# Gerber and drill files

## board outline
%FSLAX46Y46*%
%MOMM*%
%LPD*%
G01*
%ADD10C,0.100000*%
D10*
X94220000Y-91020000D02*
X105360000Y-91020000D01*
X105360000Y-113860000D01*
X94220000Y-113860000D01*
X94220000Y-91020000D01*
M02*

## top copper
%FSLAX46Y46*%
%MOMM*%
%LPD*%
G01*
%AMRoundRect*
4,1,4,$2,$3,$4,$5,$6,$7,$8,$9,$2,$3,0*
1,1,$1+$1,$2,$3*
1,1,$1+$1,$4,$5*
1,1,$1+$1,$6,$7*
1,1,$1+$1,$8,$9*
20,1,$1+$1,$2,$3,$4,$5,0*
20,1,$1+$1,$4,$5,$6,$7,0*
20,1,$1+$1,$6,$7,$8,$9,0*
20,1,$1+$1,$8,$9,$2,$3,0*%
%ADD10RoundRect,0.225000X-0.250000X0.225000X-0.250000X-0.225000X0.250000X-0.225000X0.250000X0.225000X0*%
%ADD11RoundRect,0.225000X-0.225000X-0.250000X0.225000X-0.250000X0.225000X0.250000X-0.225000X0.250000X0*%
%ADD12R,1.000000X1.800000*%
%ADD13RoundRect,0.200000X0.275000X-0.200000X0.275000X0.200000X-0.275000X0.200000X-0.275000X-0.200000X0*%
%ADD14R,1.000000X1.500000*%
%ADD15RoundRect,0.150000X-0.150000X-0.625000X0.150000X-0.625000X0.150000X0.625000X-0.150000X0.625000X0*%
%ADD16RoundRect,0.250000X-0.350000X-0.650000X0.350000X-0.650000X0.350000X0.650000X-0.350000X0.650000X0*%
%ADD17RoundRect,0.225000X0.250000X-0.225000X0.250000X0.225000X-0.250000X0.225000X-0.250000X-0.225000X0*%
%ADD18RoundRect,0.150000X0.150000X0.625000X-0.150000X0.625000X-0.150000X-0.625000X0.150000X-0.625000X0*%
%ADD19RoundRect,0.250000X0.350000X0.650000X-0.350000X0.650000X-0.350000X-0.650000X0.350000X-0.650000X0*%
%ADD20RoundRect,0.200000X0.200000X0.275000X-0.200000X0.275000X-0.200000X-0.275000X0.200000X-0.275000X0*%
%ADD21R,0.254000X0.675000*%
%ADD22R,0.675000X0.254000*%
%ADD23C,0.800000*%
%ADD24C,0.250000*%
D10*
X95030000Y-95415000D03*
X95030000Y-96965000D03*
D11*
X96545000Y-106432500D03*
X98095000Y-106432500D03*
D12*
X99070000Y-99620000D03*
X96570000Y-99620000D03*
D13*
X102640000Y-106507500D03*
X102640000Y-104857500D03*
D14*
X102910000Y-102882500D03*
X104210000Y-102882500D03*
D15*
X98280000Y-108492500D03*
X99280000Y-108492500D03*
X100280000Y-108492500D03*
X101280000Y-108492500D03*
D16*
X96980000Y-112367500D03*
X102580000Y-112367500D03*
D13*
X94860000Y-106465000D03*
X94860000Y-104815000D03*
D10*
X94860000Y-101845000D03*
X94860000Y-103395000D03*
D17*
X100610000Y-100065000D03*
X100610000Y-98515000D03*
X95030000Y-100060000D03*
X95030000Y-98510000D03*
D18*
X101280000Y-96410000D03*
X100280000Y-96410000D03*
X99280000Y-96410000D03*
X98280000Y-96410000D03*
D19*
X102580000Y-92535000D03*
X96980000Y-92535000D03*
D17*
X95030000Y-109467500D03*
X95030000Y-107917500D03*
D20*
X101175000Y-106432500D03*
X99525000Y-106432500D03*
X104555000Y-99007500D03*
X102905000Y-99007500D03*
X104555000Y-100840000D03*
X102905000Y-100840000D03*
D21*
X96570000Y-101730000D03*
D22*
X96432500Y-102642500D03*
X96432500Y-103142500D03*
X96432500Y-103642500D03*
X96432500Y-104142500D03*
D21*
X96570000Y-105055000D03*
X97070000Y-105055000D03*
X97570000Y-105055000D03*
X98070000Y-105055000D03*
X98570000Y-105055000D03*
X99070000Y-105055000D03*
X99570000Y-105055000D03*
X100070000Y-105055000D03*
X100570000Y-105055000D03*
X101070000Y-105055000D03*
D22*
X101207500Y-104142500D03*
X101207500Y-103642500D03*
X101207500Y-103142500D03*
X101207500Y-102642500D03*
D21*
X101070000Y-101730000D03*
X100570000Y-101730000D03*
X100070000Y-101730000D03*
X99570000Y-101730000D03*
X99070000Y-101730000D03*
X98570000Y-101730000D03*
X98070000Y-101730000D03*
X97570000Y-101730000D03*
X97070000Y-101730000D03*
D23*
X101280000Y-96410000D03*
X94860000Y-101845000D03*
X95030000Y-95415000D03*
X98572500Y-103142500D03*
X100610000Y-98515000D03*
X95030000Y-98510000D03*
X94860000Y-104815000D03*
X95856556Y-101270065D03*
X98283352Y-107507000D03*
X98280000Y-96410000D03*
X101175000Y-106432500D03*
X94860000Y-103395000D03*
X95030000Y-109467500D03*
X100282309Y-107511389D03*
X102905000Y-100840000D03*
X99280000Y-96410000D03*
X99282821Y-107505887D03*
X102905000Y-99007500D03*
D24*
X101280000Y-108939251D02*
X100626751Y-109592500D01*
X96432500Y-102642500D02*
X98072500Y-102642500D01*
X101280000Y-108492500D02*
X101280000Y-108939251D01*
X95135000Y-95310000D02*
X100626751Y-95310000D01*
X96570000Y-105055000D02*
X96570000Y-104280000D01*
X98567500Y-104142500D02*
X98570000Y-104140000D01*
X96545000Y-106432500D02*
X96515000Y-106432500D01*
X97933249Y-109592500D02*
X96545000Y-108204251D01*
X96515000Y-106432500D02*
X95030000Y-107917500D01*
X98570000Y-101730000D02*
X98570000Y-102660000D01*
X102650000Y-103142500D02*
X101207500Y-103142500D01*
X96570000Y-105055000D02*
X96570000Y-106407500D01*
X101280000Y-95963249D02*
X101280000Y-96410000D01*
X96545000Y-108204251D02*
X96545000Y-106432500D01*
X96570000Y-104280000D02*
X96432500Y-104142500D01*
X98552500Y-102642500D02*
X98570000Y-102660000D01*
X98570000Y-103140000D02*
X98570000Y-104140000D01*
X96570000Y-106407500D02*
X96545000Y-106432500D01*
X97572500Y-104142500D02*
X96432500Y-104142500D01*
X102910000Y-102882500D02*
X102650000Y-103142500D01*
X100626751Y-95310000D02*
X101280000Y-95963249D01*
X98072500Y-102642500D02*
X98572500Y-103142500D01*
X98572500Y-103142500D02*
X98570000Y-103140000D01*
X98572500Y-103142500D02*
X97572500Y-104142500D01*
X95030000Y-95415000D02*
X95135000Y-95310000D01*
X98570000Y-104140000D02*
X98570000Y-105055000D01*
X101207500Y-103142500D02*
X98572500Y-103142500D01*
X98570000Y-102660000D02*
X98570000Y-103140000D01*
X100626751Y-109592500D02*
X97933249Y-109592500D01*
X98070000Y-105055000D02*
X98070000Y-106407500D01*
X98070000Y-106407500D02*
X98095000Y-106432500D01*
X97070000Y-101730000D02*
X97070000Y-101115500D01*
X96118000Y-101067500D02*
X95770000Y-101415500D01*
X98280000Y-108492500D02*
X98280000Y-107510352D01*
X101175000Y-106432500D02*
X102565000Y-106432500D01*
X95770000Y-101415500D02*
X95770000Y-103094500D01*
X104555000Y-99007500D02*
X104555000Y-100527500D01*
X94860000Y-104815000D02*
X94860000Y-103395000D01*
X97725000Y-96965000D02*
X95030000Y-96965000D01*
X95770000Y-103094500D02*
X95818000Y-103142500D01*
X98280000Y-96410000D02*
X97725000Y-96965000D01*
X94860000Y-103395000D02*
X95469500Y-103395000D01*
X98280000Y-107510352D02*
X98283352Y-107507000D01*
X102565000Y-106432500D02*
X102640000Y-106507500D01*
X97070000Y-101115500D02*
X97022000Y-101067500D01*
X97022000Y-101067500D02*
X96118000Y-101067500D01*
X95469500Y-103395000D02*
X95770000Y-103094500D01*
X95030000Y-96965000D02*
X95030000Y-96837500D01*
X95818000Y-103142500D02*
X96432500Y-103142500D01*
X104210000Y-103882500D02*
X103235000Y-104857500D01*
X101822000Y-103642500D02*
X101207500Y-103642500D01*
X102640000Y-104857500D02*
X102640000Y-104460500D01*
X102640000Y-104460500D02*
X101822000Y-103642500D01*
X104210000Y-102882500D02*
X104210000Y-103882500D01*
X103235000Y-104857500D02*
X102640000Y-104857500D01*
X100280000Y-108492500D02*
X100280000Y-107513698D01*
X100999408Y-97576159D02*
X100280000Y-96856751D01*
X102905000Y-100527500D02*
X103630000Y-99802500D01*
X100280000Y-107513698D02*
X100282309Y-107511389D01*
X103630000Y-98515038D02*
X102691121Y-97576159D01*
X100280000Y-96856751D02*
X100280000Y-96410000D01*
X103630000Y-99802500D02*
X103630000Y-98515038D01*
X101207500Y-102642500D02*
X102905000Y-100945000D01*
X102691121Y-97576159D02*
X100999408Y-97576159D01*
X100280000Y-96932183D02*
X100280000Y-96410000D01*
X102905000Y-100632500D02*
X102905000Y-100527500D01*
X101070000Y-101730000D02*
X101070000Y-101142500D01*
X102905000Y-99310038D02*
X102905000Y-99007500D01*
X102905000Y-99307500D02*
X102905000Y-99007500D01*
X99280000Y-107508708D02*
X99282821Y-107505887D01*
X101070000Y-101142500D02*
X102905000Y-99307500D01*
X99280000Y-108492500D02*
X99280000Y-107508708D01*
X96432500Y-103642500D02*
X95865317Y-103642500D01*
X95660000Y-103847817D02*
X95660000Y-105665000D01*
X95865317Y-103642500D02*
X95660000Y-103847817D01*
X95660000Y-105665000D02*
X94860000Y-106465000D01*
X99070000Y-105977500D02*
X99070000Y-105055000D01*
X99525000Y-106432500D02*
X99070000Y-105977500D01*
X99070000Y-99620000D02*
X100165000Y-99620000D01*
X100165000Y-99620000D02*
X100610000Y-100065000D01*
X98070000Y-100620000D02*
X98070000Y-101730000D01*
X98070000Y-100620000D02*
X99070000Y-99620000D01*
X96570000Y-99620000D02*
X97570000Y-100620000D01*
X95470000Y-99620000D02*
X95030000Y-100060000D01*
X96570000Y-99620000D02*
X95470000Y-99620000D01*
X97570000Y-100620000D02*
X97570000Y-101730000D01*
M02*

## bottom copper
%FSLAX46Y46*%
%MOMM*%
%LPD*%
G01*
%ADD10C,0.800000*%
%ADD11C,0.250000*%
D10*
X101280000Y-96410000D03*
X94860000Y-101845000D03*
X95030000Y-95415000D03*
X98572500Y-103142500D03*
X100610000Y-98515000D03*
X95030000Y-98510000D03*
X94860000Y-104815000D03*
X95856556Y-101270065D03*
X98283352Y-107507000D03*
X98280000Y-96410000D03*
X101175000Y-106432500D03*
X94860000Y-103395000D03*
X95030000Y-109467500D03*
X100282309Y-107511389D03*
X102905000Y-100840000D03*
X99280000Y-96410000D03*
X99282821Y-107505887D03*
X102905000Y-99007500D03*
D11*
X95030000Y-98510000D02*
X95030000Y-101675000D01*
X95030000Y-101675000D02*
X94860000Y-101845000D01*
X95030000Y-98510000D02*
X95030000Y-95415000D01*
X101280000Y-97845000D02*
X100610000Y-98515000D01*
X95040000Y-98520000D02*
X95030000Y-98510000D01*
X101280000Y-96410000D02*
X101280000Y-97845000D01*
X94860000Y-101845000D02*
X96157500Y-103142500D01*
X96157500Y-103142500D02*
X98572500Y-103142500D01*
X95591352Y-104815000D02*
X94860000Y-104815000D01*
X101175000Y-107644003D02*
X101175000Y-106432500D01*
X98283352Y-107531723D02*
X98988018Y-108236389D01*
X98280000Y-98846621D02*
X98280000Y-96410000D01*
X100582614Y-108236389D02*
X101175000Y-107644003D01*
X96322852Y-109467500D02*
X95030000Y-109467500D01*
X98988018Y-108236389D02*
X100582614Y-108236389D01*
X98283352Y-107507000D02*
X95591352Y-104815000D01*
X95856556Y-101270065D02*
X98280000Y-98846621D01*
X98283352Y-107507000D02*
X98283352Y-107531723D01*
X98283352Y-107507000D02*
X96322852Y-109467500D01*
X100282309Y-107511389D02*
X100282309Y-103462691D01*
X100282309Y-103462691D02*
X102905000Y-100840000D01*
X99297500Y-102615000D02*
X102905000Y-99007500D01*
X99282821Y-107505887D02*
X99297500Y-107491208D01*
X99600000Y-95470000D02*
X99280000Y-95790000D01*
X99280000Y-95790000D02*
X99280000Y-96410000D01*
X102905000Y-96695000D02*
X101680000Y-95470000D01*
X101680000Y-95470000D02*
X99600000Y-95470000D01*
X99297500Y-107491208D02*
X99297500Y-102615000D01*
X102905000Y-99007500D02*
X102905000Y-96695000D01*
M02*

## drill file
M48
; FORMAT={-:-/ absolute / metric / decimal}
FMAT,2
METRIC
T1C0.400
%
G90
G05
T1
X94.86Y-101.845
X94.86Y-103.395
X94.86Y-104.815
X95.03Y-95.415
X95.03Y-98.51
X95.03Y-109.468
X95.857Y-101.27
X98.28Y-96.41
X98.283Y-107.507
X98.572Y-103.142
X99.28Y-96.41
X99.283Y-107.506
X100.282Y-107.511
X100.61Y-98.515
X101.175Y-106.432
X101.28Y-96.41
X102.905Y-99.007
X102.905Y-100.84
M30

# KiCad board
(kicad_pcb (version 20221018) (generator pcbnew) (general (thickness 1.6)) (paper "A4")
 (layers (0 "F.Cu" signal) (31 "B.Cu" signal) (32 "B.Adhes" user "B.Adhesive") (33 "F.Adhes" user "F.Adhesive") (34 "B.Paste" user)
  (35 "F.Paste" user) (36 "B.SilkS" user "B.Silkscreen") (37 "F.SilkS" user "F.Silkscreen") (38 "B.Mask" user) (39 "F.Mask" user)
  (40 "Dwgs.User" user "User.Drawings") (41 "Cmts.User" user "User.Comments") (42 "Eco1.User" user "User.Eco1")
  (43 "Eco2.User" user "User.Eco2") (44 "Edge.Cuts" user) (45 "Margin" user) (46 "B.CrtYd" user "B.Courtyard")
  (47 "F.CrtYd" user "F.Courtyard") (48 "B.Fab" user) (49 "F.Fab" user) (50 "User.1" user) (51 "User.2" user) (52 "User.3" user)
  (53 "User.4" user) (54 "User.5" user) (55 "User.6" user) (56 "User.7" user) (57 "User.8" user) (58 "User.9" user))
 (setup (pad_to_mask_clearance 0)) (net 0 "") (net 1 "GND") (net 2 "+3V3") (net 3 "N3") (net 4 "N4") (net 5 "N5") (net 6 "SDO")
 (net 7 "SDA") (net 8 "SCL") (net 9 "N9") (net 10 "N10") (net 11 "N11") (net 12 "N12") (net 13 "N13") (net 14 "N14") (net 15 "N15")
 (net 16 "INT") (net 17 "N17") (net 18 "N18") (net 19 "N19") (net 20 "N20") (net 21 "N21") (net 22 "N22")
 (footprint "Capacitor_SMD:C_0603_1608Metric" (layer "F.Cu") (at 95.03 96.19 -90)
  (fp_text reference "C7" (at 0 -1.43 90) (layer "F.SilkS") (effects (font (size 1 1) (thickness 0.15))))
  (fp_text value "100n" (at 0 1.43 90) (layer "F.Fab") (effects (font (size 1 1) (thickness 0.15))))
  (pad "1" smd roundrect (at -0.775 0 270) (size 0.9 0.95) (layers "F.Cu" "F.Paste" "F.Mask") (roundrect_rratio 0.25) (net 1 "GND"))
  (pad "2" smd roundrect (at 0.775 0 270) (size 0.9 0.95) (layers "F.Cu" "F.Paste" "F.Mask") (roundrect_rratio 0.25) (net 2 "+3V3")))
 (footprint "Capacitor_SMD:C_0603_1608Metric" (layer "F.Cu") (at 97.32 106.4325)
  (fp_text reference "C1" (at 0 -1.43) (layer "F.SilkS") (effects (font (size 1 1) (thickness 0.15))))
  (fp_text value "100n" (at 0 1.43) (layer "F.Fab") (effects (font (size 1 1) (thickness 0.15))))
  (pad "1" smd roundrect (at -0.775 0) (size 0.9 0.95) (layers "F.Cu" "F.Paste" "F.Mask") (roundrect_rratio 0.25) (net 1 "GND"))
  (pad "2" smd roundrect (at 0.775 0) (size 0.9 0.95) (layers "F.Cu" "F.Paste" "F.Mask") (roundrect_rratio 0.25) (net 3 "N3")))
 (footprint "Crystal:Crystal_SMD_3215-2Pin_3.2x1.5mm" (layer "F.Cu") (at 97.82 99.62)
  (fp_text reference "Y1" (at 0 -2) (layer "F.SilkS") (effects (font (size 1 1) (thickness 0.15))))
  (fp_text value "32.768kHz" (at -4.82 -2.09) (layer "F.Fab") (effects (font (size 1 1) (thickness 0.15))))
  (pad "1" smd rect (at 1.25 0) (size 1 1.8) (layers "F.Cu" "F.Paste" "F.Mask") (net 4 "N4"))
  (pad "2" smd rect (at -1.25 0) (size 1 1.8) (layers "F.Cu" "F.Paste" "F.Mask") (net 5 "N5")))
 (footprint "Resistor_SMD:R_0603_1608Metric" (layer "F.Cu") (at 102.64 105.6825 90)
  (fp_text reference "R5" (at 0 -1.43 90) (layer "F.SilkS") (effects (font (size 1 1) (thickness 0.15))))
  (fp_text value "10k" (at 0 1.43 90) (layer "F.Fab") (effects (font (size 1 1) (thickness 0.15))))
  (pad "1" smd roundrect (at -0.825 0 90) (size 0.8 0.95) (layers "F.Cu" "F.Paste" "F.Mask") (roundrect_rratio 0.25) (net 2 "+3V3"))
  (pad "2" smd roundrect (at 0.825 0 90) (size 0.8 0.95) (layers "F.Cu" "F.Paste" "F.Mask") (roundrect_rratio 0.25) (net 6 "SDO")))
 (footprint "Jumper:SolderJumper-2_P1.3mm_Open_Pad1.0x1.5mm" (layer "F.Cu") (at 103.56 102.8825)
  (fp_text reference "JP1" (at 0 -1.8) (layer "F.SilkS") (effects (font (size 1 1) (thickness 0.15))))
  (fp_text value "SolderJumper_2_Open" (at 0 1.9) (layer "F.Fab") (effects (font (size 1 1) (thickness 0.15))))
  (pad "1" smd rect (at -0.65 0) (size 1 1.5) (layers "F.Cu" "F.Mask") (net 1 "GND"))
  (pad "2" smd rect (at 0.65 0) (size 1 1.5) (layers "F.Cu" "F.Mask") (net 6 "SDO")))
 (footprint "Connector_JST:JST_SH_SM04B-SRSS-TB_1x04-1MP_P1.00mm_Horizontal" (layer "F.Cu") (at 99.78 110.4925)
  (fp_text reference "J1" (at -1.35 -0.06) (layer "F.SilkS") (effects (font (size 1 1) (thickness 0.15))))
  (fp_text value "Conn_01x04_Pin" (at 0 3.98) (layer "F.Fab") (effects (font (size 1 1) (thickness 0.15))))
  (pad "1" smd roundrect (at -1.5 -2) (size 0.6 1.55) (layers "F.Cu" "F.Paste" "F.Mask") (roundrect_rratio 0.25) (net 2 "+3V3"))
  (pad "2" smd roundrect (at -0.5 -2) (size 0.6 1.55) (layers "F.Cu" "F.Paste" "F.Mask") (roundrect_rratio 0.25) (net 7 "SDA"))
  (pad "3" smd roundrect (at 0.5 -2) (size 0.6 1.55) (layers "F.Cu" "F.Paste" "F.Mask") (roundrect_rratio 0.25) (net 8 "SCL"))
  (pad "4" smd roundrect (at 1.5 -2) (size 0.6 1.55) (layers "F.Cu" "F.Paste" "F.Mask") (roundrect_rratio 0.25) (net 1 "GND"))
  (pad "MP" smd roundrect (at -2.8 1.875) (size 1.2 1.8) (layers "F.Cu" "F.Paste" "F.Mask") (roundrect_rratio 0.208333))
  (pad "MP" smd roundrect (at 2.8 1.875) (size 1.2 1.8) (layers "F.Cu" "F.Paste" "F.Mask") (roundrect_rratio 0.208333)))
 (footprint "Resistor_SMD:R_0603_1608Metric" (layer "F.Cu") (at 94.86 105.64 90)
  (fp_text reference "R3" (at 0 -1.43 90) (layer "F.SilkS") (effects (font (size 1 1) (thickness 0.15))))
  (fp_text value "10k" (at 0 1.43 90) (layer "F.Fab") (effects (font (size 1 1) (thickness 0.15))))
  (pad "1" smd roundrect (at -0.825 0 90) (size 0.8 0.95) (layers "F.Cu" "F.Paste" "F.Mask") (roundrect_rratio 0.25) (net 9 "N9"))
  (pad "2" smd roundrect (at 0.825 0 90) (size 0.8 0.95) (layers "F.Cu" "F.Paste" "F.Mask") (roundrect_rratio 0.25) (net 2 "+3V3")))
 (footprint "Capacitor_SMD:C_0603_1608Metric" (layer "F.Cu") (at 94.86 102.62 -90)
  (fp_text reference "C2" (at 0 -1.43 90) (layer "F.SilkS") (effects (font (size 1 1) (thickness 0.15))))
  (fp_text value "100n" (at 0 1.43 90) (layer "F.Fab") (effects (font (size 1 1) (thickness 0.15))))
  (pad "1" smd roundrect (at -0.775 0 270) (size 0.9 0.95) (layers "F.Cu" "F.Paste" "F.Mask") (roundrect_rratio 0.25) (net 1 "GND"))
  (pad "2" smd roundrect (at 0.775 0 270) (size 0.9 0.95) (layers "F.Cu" "F.Paste" "F.Mask") (roundrect_rratio 0.25) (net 2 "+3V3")))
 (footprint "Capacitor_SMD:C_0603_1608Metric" (layer "F.Cu") (at 100.61 99.29 90)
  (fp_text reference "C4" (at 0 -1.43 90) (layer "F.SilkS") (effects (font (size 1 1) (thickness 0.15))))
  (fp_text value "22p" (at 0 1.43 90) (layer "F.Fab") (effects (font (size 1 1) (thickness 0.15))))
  (pad "1" smd roundrect (at -0.775 0 90) (size 0.9 0.95) (layers "F.Cu" "F.Paste" "F.Mask") (roundrect_rratio 0.25) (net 4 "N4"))
  (pad "2" smd roundrect (at 0.775 0 90) (size 0.9 0.95) (layers "F.Cu" "F.Paste" "F.Mask") (roundrect_rratio 0.25) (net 1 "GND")))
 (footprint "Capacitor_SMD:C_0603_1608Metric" (layer "F.Cu") (at 95.03 99.285 90)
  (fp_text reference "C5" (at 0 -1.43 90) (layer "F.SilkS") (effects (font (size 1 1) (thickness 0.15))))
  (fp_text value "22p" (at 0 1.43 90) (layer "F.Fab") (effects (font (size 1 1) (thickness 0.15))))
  (pad "1" smd roundrect (at -0.775 0 90) (size 0.9 0.95) (layers "F.Cu" "F.Paste" "F.Mask") (roundrect_rratio 0.25) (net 5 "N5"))
  (pad "2" smd roundrect (at 0.775 0 90) (size 0.9 0.95) (layers "F.Cu" "F.Paste" "F.Mask") (roundrect_rratio 0.25) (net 1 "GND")))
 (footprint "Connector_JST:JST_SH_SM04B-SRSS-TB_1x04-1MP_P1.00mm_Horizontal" (layer "F.Cu") (at 99.78 94.41 180)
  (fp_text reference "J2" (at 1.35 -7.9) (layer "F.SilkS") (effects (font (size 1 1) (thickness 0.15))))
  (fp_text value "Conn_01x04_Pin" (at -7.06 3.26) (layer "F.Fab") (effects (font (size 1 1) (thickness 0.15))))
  (pad "1" smd roundrect (at -1.5 -2 180) (size 0.6 1.55) (layers "F.Cu" "F.Paste" "F.Mask") (roundrect_rratio 0.25) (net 1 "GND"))
  (pad "2" smd roundrect (at -0.5 -2 180) (size 0.6 1.55) (layers "F.Cu" "F.Paste" "F.Mask") (roundrect_rratio 0.25) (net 8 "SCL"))
  (pad "3" smd roundrect (at 0.5 -2 180) (size 0.6 1.55) (layers "F.Cu" "F.Paste" "F.Mask") (roundrect_rratio 0.25) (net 7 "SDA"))
  (pad "4" smd roundrect (at 1.5 -2 180) (size 0.6 1.55) (layers "F.Cu" "F.Paste" "F.Mask") (roundrect_rratio 0.25) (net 2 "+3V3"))
  (pad "MP" smd roundrect (at -2.8 1.875 180) (size 1.2 1.8) (layers "F.Cu" "F.Paste" "F.Mask") (roundrect_rratio 0.208333))
  (pad "MP" smd roundrect (at 2.8 1.875 180) (size 1.2 1.8) (layers "F.Cu" "F.Paste" "F.Mask") (roundrect_rratio 0.208333)))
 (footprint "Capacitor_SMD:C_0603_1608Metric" (layer "F.Cu") (at 95.03 108.6925 90)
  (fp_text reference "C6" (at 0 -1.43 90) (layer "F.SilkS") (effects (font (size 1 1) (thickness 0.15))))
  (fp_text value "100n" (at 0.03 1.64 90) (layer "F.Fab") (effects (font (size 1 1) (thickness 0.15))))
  (pad "1" smd roundrect (at -0.775 0 90) (size 0.9 0.95) (layers "F.Cu" "F.Paste" "F.Mask") (roundrect_rratio 0.25) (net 2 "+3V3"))
  (pad "2" smd roundrect (at 0.775 0 90) (size 0.9 0.95) (layers "F.Cu" "F.Paste" "F.Mask") (roundrect_rratio 0.25) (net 1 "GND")))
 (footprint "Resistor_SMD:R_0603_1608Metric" (layer "F.Cu") (at 100.35 106.4325 180)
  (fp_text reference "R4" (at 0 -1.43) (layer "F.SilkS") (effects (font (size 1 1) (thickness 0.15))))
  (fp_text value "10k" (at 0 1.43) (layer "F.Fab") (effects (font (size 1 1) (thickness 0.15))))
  (pad "1" smd roundrect (at -0.825 0 180) (size 0.8 0.95) (layers "F.Cu" "F.Paste" "F.Mask") (roundrect_rratio 0.25) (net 2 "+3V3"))
  (pad "2" smd roundrect (at 0.825 0 180) (size 0.8 0.95) (layers "F.Cu" "F.Paste" "F.Mask") (roundrect_rratio 0.25) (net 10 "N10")))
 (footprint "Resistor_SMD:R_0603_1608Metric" (layer "F.Cu") (at 103.73 99.0075 180)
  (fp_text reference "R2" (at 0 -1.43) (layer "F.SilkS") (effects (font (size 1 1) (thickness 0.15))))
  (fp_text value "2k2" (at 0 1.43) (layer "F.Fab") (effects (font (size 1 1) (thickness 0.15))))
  (pad "1" smd roundrect (at -0.825 0 180) (size 0.8 0.95) (layers "F.Cu" "F.Paste" "F.Mask") (roundrect_rratio 0.25) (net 2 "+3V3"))
  (pad "2" smd roundrect (at 0.825 0 180) (size 0.8 0.95) (layers "F.Cu" "F.Paste" "F.Mask") (roundrect_rratio 0.25) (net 7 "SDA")))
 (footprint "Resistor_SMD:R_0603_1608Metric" (layer "F.Cu") (at 103.73 100.84 180)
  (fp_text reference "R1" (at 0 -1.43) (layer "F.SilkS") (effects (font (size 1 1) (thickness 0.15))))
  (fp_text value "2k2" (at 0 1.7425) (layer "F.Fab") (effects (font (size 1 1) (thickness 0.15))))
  (pad "1" smd roundrect (at -0.825 0 180) (size 0.8 0.95) (layers "F.Cu" "F.Paste" "F.Mask") (roundrect_rratio 0.25) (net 2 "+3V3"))
  (pad "2" smd roundrect (at 0.825 0 180) (size 0.8 0.95) (layers "F.Cu" "F.Paste" "F.Mask") (roundrect_rratio 0.25) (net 8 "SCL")))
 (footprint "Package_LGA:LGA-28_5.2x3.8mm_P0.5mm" (layer "F.Cu") (at 98.82 103.3925)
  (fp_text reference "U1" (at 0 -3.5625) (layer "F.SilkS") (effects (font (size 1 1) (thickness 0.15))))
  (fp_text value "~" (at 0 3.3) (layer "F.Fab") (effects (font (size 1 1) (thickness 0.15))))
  (pad "1" smd rect (at -2.25 -1.6625) (size 0.254 0.675) (layers "F.Cu" "F.Paste" "F.Mask") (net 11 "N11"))
  (pad "2" smd rect (at -2.3875 -0.75 90) (size 0.254 0.675) (layers "F.Cu" "F.Paste" "F.Mask") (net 1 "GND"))
  (pad "3" smd rect (at -2.3875 -0.25 90) (size 0.254 0.675) (layers "F.Cu" "F.Paste" "F.Mask") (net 2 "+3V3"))
  (pad "4" smd rect (at -2.3875 0.25 90) (size 0.254 0.675) (layers "F.Cu" "F.Paste" "F.Mask") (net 9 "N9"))
  (pad "5" smd rect (at -2.3875 0.75 90) (size 0.254 0.675) (layers "F.Cu" "F.Paste" "F.Mask") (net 1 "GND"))
  (pad "6" smd rect (at -2.25 1.6625) (size 0.254 0.675) (layers "F.Cu" "F.Paste" "F.Mask") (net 1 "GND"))
  (pad "7" smd rect (at -1.75 1.6625) (size 0.254 0.675) (layers "F.Cu" "F.Paste" "F.Mask") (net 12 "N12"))
  (pad "8" smd rect (at -1.25 1.6625) (size 0.254 0.675) (layers "F.Cu" "F.Paste" "F.Mask") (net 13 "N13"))
  (pad "9" smd rect (at -0.75 1.6625) (size 0.254 0.675) (layers "F.Cu" "F.Paste" "F.Mask") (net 3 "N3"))
  (pad "10" smd rect (at -0.25 1.6625) (size 0.254 0.675) (layers "F.Cu" "F.Paste" "F.Mask") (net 1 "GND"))
  (pad "11" smd rect (at 0.25 1.6625) (size 0.254 0.675) (layers "F.Cu" "F.Paste" "F.Mask") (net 10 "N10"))
  (pad "12" smd rect (at 0.75 1.6625) (size 0.254 0.675) (layers "F.Cu" "F.Paste" "F.Mask") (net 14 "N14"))
  (pad "13" smd rect (at 1.25 1.6625) (size 0.254 0.675) (layers "F.Cu" "F.Paste" "F.Mask") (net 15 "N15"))
  (pad "14" smd rect (at 1.75 1.6625) (size 0.254 0.675) (layers "F.Cu" "F.Paste" "F.Mask") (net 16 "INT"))
  (pad "15" smd rect (at 2.25 1.6625) (size 0.254 0.675) (layers "F.Cu" "F.Paste" "F.Mask") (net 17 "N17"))
  (pad "16" smd rect (at 2.3875 0.75 90) (size 0.254 0.675) (layers "F.Cu" "F.Paste" "F.Mask") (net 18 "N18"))
  (pad "17" smd rect (at 2.3875 0.25 90) (size 0.254 0.675) (layers "F.Cu" "F.Paste" "F.Mask") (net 6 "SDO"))
  (pad "18" smd rect (at 2.3875 -0.25 90) (size 0.254 0.675) (layers "F.Cu" "F.Paste" "F.Mask") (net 1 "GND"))
  (pad "19" smd rect (at 2.3875 -0.75 90) (size 0.254 0.675) (layers "F.Cu" "F.Paste" "F.Mask") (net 8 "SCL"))
  (pad "20" smd rect (at 2.25 -1.6625) (size 0.254 0.675) (layers "F.Cu" "F.Paste" "F.Mask") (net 7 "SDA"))
  (pad "21" smd rect (at 1.75 -1.6625) (size 0.254 0.675) (layers "F.Cu" "F.Paste" "F.Mask") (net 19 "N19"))
  (pad "22" smd rect (at 1.25 -1.6625) (size 0.254 0.675) (layers "F.Cu" "F.Paste" "F.Mask") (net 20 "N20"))
  (pad "23" smd rect (at 0.75 -1.6625) (size 0.254 0.675) (layers "F.Cu" "F.Paste" "F.Mask") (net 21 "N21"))
  (pad "24" smd rect (at 0.25 -1.6625) (size 0.254 0.675) (layers "F.Cu" "F.Paste" "F.Mask") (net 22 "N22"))
  (pad "25" smd rect (at -0.25 -1.6625) (size 0.254 0.675) (layers "F.Cu" "F.Paste" "F.Mask") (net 1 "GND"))
  (pad "26" smd rect (at -0.75 -1.6625) (size 0.254 0.675) (layers "F.Cu" "F.Paste" "F.Mask") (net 4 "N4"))
  (pad "27" smd rect (at -1.25 -1.6625) (size 0.254 0.675) (layers "F.Cu" "F.Paste" "F.Mask") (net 5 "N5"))
  (pad "28" smd rect (at -1.75 -1.6625) (size 0.254 0.675) (layers "F.Cu" "F.Paste" "F.Mask") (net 2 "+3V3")))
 (gr_rect (start 94.22 91.02) (end 105.36 113.86) (stroke (width 0.1) (type default)) (fill none) (layer "Edge.Cuts"))
 (segment (start 101.28 108.939251) (end 100.626751 109.5925) (width 0.25) (layer "F.Cu") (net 1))
 (segment (start 96.4325 102.6425) (end 98.0725 102.6425) (width 0.25) (layer "F.Cu") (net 1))
 (segment (start 101.28 108.4925) (end 101.28 108.939251) (width 0.25) (layer "F.Cu") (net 1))
 (segment (start 95.135 95.31) (end 100.626751 95.31) (width 0.25) (layer "F.Cu") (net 1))
 (segment (start 96.57 105.055) (end 96.57 104.28) (width 0.25) (layer "F.Cu") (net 1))
 (segment (start 98.5675 104.1425) (end 98.57 104.14) (width 0.25) (layer "F.Cu") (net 1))
 (segment (start 96.545 106.4325) (end 96.515 106.4325) (width 0.25) (layer "F.Cu") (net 1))
 (segment (start 97.933249 109.5925) (end 96.545 108.204251) (width 0.25) (layer "F.Cu") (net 1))
 (segment (start 96.515 106.4325) (end 95.03 107.9175) (width 0.25) (layer "F.Cu") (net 1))
 (segment (start 98.57 101.73) (end 98.57 102.66) (width 0.25) (layer "F.Cu") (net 1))
 (segment (start 102.65 103.1425) (end 101.2075 103.1425) (width 0.25) (layer "F.Cu") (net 1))
 (segment (start 96.57 105.055) (end 96.57 106.4075) (width 0.25) (layer "F.Cu") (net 1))
 (segment (start 101.28 95.963249) (end 101.28 96.41) (width 0.25) (layer "F.Cu") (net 1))
 (segment (start 96.545 108.204251) (end 96.545 106.4325) (width 0.25) (layer "F.Cu") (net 1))
 (segment (start 96.57 104.28) (end 96.4325 104.1425) (width 0.25) (layer "F.Cu") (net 1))
 (segment (start 98.5525 102.6425) (end 98.57 102.66) (width 0.25) (layer "F.Cu") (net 1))
 (segment (start 98.57 103.14) (end 98.57 104.14) (width 0.25) (layer "F.Cu") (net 1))
 (segment (start 96.57 106.4075) (end 96.545 106.4325) (width 0.25) (layer "F.Cu") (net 1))
 (segment (start 97.5725 104.1425) (end 96.4325 104.1425) (width 0.25) (layer "F.Cu") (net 1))
 (segment (start 102.91 102.8825) (end 102.65 103.1425) (width 0.25) (layer "F.Cu") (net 1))
 (segment (start 100.626751 95.31) (end 101.28 95.963249) (width 0.25) (layer "F.Cu") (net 1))
 (segment (start 98.0725 102.6425) (end 98.5725 103.1425) (width 0.25) (layer "F.Cu") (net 1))
 (segment (start 98.5725 103.1425) (end 98.57 103.14) (width 0.25) (layer "F.Cu") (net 1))
 (segment (start 98.5725 103.1425) (end 97.5725 104.1425) (width 0.25) (layer "F.Cu") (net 1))
 (segment (start 95.03 95.415) (end 95.135 95.31) (width 0.25) (layer "F.Cu") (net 1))
 (segment (start 98.57 104.14) (end 98.57 105.055) (width 0.25) (layer "F.Cu") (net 1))
 (segment (start 101.2075 103.1425) (end 98.5725 103.1425) (width 0.25) (layer "F.Cu") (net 1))
 (segment (start 98.57 102.66) (end 98.57 103.14) (width 0.25) (layer "F.Cu") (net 1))
 (segment (start 100.626751 109.5925) (end 97.933249 109.5925) (width 0.25) (layer "F.Cu") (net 1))
 (via (at 101.28 96.41) (size 0.8) (drill 0.4) (layers "F.Cu" "B.Cu") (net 1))
 (via (at 94.86 101.845) (size 0.8) (drill 0.4) (layers "F.Cu" "B.Cu") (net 1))
 (via (at 95.03 95.415) (size 0.8) (drill 0.4) (layers "F.Cu" "B.Cu") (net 1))
 (via (at 98.5725 103.1425) (size 0.8) (drill 0.4) (layers "F.Cu" "B.Cu") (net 1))
 (via (at 100.61 98.515) (size 0.8) (drill 0.4) (layers "F.Cu" "B.Cu") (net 1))
 (via (at 95.03 98.51) (size 0.8) (drill 0.4) (layers "F.Cu" "B.Cu") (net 1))
 (segment (start 95.03 98.51) (end 95.03 101.675) (width 0.25) (layer "B.Cu") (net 1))
 (segment (start 95.03 101.675) (end 94.86 101.845) (width 0.25) (layer "B.Cu") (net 1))
 (segment (start 95.03 98.51) (end 95.03 95.415) (width 0.25) (layer "B.Cu") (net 1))
 (segment (start 101.28 97.845) (end 100.61 98.515) (width 0.25) (layer "B.Cu") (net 1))
 (segment (start 95.04 98.52) (end 95.03 98.51) (width 0.25) (layer "B.Cu") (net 1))
 (segment (start 101.28 96.41) (end 101.28 97.845) (width 0.25) (layer "B.Cu") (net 1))
 (segment (start 94.86 101.845) (end 96.1575 103.1425) (width 0.25) (layer "B.Cu") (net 1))
 (segment (start 96.1575 103.1425) (end 98.5725 103.1425) (width 0.25) (layer "B.Cu") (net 1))
 (segment (start 98.07 105.055) (end 98.07 106.4075) (width 0.25) (layer "F.Cu") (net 3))
 (segment (start 98.07 106.4075) (end 98.095 106.4325) (width 0.25) (layer "F.Cu") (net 3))
 (segment (start 97.07 101.73) (end 97.07 101.1155) (width 0.25) (layer "F.Cu") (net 2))
 (segment (start 96.118 101.0675) (end 95.77 101.4155) (width 0.25) (layer "F.Cu") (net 2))
 (segment (start 98.28 108.4925) (end 98.28 107.510352) (width 0.25) (layer "F.Cu") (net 2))
 (segment (start 101.175 106.4325) (end 102.565 106.4325) (width 0.25) (layer "F.Cu") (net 2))
 (segment (start 95.77 101.4155) (end 95.77 103.0945) (width 0.25) (layer "F.Cu") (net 2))
 (segment (start 104.555 99.0075) (end 104.555 100.5275) (width 0.25) (layer "F.Cu") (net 2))
 (segment (start 94.86 104.815) (end 94.86 103.395) (width 0.25) (layer "F.Cu") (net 2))
 (segment (start 97.725 96.965) (end 95.03 96.965) (width 0.25) (layer "F.Cu") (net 2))
 (segment (start 95.77 103.0945) (end 95.818 103.1425) (width 0.25) (layer "F.Cu") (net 2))
 (segment (start 98.28 96.41) (end 97.725 96.965) (width 0.25) (layer "F.Cu") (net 2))
 (segment (start 94.86 103.395) (end 95.4695 103.395) (width 0.25) (layer "F.Cu") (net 2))
 (segment (start 98.28 107.510352) (end 98.283352 107.507) (width 0.25) (layer "F.Cu") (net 2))
 (segment (start 102.565 106.4325) (end 102.64 106.5075) (width 0.25) (layer "F.Cu") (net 2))
 (segment (start 97.07 101.1155) (end 97.022 101.0675) (width 0.25) (layer "F.Cu") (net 2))
 (segment (start 97.022 101.0675) (end 96.118 101.0675) (width 0.25) (layer "F.Cu") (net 2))
 (segment (start 95.4695 103.395) (end 95.77 103.0945) (width 0.25) (layer "F.Cu") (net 2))
 (segment (start 95.03 96.965) (end 95.03 96.8375) (width 0.25) (layer "F.Cu") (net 2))
 (segment (start 95.818 103.1425) (end 96.4325 103.1425) (width 0.25) (layer "F.Cu") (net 2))
 (via (at 94.86 104.815) (size 0.8) (drill 0.4) (layers "F.Cu" "B.Cu") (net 2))
 (via (at 95.856556 101.270065) (size 0.8) (drill 0.4) (layers "F.Cu" "B.Cu") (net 2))
 (via (at 98.283352 107.507) (size 0.8) (drill 0.4) (layers "F.Cu" "B.Cu") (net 2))
 (via (at 98.28 96.41) (size 0.8) (drill 0.4) (layers "F.Cu" "B.Cu") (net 2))
 (via (at 101.175 106.4325) (size 0.8) (drill 0.4) (layers "F.Cu" "B.Cu") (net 2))
 (via (at 94.86 103.395) (size 0.8) (drill 0.4) (layers "F.Cu" "B.Cu") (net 2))
 (via (at 95.03 109.4675) (size 0.8) (drill 0.4) (layers "F.Cu" "B.Cu") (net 2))
 (segment (start 95.591352 104.815) (end 94.86 104.815) (width 0.25) (layer "B.Cu") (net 2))
 (segment (start 101.175 107.644003) (end 101.175 106.4325) (width 0.25) (layer "B.Cu") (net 2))
 (segment (start 98.283352 107.531723) (end 98.988018 108.236389) (width 0.25) (layer "B.Cu") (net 2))
 (segment (start 98.28 98.846621) (end 98.28 96.41) (width 0.25) (layer "B.Cu") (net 2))
 (segment (start 100.582614 108.236389) (end 101.175 107.644003) (width 0.25) (layer "B.Cu") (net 2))
 (segment (start 96.322852 109.4675) (end 95.03 109.4675) (width 0.25) (layer "B.Cu") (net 2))
 (segment (start 98.988018 108.236389) (end 100.582614 108.236389) (width 0.25) (layer "B.Cu") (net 2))
 (segment (start 98.283352 107.507) (end 95.591352 104.815) (width 0.25) (layer "B.Cu") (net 2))
 (segment (start 95.856556 101.270065) (end 98.28 98.846621) (width 0.25) (layer "B.Cu") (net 2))
 (segment (start 98.283352 107.507) (end 98.283352 107.531723) (width 0.25) (layer "B.Cu") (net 2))
 (segment (start 98.283352 107.507) (end 96.322852 109.4675) (width 0.25) (layer "B.Cu") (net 2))
 (segment (start 104.21 103.8825) (end 103.235 104.8575) (width 0.25) (layer "F.Cu") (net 6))
 (segment (start 101.822 103.6425) (end 101.2075 103.6425) (width 0.25) (layer "F.Cu") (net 6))
 (segment (start 102.64 104.8575) (end 102.64 104.4605) (width 0.25) (layer "F.Cu") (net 6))
 (segment (start 102.64 104.4605) (end 101.822 103.6425) (width 0.25) (layer "F.Cu") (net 6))
 (segment (start 104.21 102.8825) (end 104.21 103.8825) (width 0.25) (layer "F.Cu") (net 6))
 (segment (start 103.235 104.8575) (end 102.64 104.8575) (width 0.25) (layer "F.Cu") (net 6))
 (segment (start 100.28 108.4925) (end 100.28 107.513698) (width 0.25) (layer "F.Cu") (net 8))
 (segment (start 100.999408 97.576159) (end 100.28 96.856751) (width 0.25) (layer "F.Cu") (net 8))
 (segment (start 102.905 100.5275) (end 103.63 99.8025) (width 0.25) (layer "F.Cu") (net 8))
 (segment (start 100.28 107.513698) (end 100.282309 107.511389) (width 0.25) (layer "F.Cu") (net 8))
 (segment (start 103.63 98.515038) (end 102.691121 97.576159) (width 0.25) (layer "F.Cu") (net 8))
 (segment (start 100.28 96.856751) (end 100.28 96.41) (width 0.25) (layer "F.Cu") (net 8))
 (segment (start 103.63 99.8025) (end 103.63 98.515038) (width 0.25) (layer "F.Cu") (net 8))
 (segment (start 101.2075 102.6425) (end 102.905 100.945) (width 0.25) (layer "F.Cu") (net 8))
 (segment (start 102.691121 97.576159) (end 100.999408 97.576159) (width 0.25) (layer "F.Cu") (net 8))
 (segment (start 100.28 96.932183) (end 100.28 96.41) (width 0.25) (layer "F.Cu") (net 8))
 (segment (start 102.905 100.6325) (end 102.905 100.5275) (width 0.25) (layer "F.Cu") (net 8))
 (via (at 100.282309 107.511389) (size 0.8) (drill 0.4) (layers "F.Cu" "B.Cu") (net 8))
 (via (at 102.905 100.84) (size 0.8) (drill 0.4) (layers "F.Cu" "B.Cu") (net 8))
 (segment (start 100.282309 107.511389) (end 100.282309 103.462691) (width 0.25) (layer "B.Cu") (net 8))
 (segment (start 100.282309 103.462691) (end 102.905 100.84) (width 0.25) (layer "B.Cu") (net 8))
 (segment (start 101.07 101.73) (end 101.07 101.1425) (width 0.25) (layer "F.Cu") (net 7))
 (segment (start 102.905 99.310038) (end 102.905 99.0075) (width 0.25) (layer "F.Cu") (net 7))
 (segment (start 102.905 99.3075) (end 102.905 99.0075) (width 0.25) (layer "F.Cu") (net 7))
 (segment (start 99.28 107.508708) (end 99.282821 107.505887) (width 0.25) (layer "F.Cu") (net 7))
 (segment (start 101.07 101.1425) (end 102.905 99.3075) (width 0.25) (layer "F.Cu") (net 7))
 (segment (start 99.28 108.4925) (end 99.28 107.508708) (width 0.25) (layer "F.Cu") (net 7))
 (via (at 99.28 96.41) (size 0.8) (drill 0.4) (layers "F.Cu" "B.Cu") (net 7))
 (via (at 99.282821 107.505887) (size 0.8) (drill 0.4) (layers "F.Cu" "B.Cu") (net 7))
 (via (at 102.905 99.0075) (size 0.8) (drill 0.4) (layers "F.Cu" "B.Cu") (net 7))
 (segment (start 99.2975 102.615) (end 102.905 99.0075) (width 0.25) (layer "B.Cu") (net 7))
 (segment (start 99.282821 107.505887) (end 99.2975 107.491208) (width 0.25) (layer "B.Cu") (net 7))
 (segment (start 99.6 95.47) (end 99.28 95.79) (width 0.25) (layer "B.Cu") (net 7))
 (segment (start 99.28 95.79) (end 99.28 96.41) (width 0.25) (layer "B.Cu") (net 7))
 (segment (start 102.905 96.695) (end 101.68 95.47) (width 0.25) (layer "B.Cu") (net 7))
 (segment (start 101.68 95.47) (end 99.6 95.47) (width 0.25) (layer "B.Cu") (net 7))
 (segment (start 99.2975 107.491208) (end 99.2975 102.615) (width 0.25) (layer "B.Cu") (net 7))
 (segment (start 102.905 99.0075) (end 102.905 96.695) (width 0.25) (layer "B.Cu") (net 7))
 (segment (start 96.4325 103.6425) (end 95.865317 103.6425) (width 0.25) (layer "F.Cu") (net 9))
 (segment (start 95.66 103.847817) (end 95.66 105.665) (width 0.25) (layer "F.Cu") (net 9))
 (segment (start 95.865317 103.6425) (end 95.66 103.847817) (width 0.25) (layer "F.Cu") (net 9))
 (segment (start 95.66 105.665) (end 94.86 106.465) (width 0.25) (layer "F.Cu") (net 9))
 (segment (start 99.07 105.9775) (end 99.07 105.055) (width 0.25) (layer "F.Cu") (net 10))
 (segment (start 99.525 106.4325) (end 99.07 105.9775) (width 0.25) (layer "F.Cu") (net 10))
 (segment (start 99.07 99.62) (end 100.165 99.62) (width 0.25) (layer "F.Cu") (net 4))
 (segment (start 100.165 99.62) (end 100.61 100.065) (width 0.25) (layer "F.Cu") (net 4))
 (segment (start 98.07 100.62) (end 98.07 101.73) (width 0.25) (layer "F.Cu") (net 4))
 (segment (start 98.07 100.62) (end 99.07 99.62) (width 0.25) (layer "F.Cu") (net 4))
 (segment (start 96.57 99.62) (end 97.57 100.62) (width 0.25) (layer "F.Cu") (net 5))
 (segment (start 95.47 99.62) (end 95.03 100.06) (width 0.25) (layer "F.Cu") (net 5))
 (segment (start 96.57 99.62) (end 95.47 99.62) (width 0.25) (layer "F.Cu") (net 5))
 (segment (start 97.57 100.62) (end 97.57 101.73) (width 0.25) (layer "F.Cu") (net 5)))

